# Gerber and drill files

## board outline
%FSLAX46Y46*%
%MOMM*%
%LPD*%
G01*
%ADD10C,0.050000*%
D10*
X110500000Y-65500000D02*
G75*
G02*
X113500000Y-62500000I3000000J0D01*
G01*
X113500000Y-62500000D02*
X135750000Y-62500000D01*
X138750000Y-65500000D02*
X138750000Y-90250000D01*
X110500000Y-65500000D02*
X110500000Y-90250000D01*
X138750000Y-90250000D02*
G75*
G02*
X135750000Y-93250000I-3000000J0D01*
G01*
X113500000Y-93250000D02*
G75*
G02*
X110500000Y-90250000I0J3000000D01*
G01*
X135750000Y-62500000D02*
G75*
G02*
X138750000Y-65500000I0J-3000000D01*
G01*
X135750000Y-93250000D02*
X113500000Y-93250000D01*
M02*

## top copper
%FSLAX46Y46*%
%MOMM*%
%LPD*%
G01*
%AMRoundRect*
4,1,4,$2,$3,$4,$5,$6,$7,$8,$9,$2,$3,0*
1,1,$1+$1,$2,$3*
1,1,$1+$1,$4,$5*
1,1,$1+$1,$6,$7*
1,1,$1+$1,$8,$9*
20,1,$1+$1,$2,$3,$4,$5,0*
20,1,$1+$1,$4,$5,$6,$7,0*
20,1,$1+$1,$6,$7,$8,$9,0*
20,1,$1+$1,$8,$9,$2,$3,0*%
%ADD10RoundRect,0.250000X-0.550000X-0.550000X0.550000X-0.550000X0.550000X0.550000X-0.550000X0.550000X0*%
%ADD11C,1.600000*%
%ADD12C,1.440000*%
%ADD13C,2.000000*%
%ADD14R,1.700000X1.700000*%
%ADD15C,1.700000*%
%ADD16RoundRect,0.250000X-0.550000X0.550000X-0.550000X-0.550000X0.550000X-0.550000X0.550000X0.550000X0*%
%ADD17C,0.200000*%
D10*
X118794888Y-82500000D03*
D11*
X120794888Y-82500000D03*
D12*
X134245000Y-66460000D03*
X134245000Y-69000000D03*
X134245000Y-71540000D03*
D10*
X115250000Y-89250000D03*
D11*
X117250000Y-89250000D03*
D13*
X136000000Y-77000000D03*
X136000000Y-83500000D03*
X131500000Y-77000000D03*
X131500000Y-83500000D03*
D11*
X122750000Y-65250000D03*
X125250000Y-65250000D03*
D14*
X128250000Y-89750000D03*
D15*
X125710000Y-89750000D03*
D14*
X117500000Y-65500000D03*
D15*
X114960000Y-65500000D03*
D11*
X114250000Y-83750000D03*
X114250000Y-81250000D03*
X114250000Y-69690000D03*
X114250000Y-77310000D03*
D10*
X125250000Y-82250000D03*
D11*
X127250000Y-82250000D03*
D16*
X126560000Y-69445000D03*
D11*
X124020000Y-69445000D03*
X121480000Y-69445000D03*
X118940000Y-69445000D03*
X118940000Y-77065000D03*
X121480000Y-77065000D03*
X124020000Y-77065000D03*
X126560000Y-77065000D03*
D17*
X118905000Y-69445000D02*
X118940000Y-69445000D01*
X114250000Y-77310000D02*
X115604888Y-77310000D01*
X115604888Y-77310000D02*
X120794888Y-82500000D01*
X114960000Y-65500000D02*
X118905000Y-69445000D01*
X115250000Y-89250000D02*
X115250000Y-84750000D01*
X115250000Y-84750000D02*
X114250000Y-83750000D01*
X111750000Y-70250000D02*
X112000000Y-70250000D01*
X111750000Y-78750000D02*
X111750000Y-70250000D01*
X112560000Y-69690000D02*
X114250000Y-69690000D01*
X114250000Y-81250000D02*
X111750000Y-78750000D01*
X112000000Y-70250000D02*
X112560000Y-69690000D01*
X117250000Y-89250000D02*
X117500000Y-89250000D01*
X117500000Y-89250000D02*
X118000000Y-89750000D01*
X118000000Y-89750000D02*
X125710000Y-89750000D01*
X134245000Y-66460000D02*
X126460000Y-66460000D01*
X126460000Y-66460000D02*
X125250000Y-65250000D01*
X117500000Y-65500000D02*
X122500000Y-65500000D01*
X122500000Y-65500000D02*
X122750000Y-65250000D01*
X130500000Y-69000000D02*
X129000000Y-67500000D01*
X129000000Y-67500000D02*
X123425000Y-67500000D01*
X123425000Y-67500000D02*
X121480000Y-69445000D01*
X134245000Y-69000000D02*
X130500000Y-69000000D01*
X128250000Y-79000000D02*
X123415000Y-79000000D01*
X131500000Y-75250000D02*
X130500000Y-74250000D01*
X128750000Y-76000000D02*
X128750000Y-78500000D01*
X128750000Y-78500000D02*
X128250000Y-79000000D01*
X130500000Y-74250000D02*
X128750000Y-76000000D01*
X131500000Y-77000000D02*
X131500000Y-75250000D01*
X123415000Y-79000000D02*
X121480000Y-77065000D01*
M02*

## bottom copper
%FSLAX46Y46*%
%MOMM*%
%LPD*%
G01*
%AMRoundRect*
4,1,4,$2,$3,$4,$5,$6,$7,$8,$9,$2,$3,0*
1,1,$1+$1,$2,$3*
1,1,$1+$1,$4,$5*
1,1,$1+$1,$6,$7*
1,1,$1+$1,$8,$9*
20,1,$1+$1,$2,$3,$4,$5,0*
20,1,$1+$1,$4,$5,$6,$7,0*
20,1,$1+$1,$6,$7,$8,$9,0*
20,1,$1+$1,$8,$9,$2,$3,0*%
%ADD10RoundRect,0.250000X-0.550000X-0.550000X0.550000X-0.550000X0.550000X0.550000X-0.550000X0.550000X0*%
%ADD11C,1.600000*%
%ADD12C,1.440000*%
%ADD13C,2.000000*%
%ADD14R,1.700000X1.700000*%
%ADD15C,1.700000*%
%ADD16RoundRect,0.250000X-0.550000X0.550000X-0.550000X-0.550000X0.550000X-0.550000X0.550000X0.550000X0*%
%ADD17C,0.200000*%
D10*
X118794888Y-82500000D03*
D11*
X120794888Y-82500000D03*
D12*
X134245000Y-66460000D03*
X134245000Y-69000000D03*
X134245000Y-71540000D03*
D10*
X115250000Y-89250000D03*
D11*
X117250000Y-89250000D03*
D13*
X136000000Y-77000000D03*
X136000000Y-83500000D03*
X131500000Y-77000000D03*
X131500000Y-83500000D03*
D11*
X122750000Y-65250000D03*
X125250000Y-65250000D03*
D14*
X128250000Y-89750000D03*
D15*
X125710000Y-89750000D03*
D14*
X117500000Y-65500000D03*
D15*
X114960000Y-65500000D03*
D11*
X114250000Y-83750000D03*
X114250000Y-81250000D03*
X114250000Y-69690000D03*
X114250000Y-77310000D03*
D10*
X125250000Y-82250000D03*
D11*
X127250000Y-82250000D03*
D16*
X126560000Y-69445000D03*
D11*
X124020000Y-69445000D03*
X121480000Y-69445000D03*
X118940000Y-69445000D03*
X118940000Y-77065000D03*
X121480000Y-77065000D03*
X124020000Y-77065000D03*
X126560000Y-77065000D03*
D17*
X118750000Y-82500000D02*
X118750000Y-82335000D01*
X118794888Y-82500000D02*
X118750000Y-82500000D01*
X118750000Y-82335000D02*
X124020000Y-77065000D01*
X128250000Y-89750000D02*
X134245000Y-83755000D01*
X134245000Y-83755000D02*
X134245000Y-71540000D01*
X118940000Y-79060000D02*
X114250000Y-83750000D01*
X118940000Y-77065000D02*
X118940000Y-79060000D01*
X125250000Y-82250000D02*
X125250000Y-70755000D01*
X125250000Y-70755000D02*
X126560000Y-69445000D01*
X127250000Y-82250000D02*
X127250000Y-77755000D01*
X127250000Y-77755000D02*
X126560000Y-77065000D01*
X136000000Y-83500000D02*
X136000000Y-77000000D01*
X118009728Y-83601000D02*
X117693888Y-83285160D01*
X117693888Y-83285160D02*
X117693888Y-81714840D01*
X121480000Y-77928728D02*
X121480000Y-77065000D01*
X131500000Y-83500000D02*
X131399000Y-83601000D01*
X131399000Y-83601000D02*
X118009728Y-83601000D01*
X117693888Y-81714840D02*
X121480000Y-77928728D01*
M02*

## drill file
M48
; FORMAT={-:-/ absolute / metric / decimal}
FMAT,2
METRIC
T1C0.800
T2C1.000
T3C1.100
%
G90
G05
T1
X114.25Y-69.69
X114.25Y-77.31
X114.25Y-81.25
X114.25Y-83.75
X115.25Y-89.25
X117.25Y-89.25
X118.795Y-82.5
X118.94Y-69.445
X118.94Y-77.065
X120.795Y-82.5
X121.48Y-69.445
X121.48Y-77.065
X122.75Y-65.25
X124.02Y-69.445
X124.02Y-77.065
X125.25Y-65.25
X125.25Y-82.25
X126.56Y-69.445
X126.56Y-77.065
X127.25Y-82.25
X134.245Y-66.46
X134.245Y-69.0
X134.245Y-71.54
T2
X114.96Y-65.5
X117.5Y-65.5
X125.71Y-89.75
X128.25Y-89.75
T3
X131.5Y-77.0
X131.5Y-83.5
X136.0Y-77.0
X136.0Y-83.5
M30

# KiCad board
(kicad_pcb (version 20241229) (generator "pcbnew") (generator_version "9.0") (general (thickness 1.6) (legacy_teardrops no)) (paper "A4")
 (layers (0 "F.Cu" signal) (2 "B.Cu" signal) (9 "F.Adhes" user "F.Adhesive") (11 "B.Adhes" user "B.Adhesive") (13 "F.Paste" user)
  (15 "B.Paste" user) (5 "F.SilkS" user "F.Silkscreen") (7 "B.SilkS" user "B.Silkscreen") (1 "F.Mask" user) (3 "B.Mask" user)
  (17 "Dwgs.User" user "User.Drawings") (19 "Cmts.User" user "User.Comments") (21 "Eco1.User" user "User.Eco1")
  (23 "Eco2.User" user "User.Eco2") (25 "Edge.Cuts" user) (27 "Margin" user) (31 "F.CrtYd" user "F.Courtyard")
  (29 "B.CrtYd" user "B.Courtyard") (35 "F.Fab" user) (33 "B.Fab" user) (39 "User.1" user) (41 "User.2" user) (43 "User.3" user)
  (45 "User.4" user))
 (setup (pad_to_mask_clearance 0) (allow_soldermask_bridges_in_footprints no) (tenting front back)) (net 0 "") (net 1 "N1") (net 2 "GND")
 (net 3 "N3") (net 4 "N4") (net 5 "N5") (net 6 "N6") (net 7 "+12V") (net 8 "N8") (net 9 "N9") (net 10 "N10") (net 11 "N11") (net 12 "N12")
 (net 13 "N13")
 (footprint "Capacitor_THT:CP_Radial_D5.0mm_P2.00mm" (layer "F.Cu") (at 118.794888 82.5)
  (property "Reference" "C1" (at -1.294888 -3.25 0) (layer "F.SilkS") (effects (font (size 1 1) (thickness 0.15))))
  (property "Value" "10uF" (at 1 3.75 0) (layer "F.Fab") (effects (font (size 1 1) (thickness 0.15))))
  (pad "1" thru_hole roundrect (at 0 0) (size 1.6 1.6) (drill 0.8) (layers "*.Cu" "*.Mask") (remove_unused_layers no)
   (roundrect_rratio 0.15625) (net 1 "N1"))
  (pad "2" thru_hole circle (at 2 0) (size 1.6 1.6) (drill 0.8) (layers "*.Cu" "*.Mask") (remove_unused_layers no) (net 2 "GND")))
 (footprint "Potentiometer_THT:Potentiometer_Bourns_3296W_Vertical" (layer "F.Cu") (at 134.245 66.46 90)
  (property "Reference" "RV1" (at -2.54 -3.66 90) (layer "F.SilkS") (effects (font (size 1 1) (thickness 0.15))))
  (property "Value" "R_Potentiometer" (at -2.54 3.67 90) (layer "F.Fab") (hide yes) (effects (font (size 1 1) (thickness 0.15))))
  (pad "1" thru_hole circle (at 0 0 90) (size 1.44 1.44) (drill 0.8) (layers "*.Cu" "*.Mask") (remove_unused_layers no) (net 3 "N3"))
  (pad "2" thru_hole circle (at -2.54 0 90) (size 1.44 1.44) (drill 0.8) (layers "*.Cu" "*.Mask") (remove_unused_layers no) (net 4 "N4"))
  (pad "3" thru_hole circle (at -5.08 0 90) (size 1.44 1.44) (drill 0.8) (layers "*.Cu" "*.Mask") (remove_unused_layers no) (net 2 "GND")))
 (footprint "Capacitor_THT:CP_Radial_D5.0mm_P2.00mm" (layer "F.Cu") (at 115.25 89.25)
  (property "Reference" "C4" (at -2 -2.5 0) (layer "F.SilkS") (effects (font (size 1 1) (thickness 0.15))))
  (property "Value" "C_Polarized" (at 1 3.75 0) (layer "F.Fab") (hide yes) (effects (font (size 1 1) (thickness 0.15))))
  (pad "1" thru_hole roundrect (at 0 0) (size 1.6 1.6) (drill 0.8) (layers "*.Cu" "*.Mask") (remove_unused_layers no)
   (roundrect_rratio 0.15625) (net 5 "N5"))
  (pad "2" thru_hole circle (at 2 0) (size 1.6 1.6) (drill 0.8) (layers "*.Cu" "*.Mask") (remove_unused_layers no) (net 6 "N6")))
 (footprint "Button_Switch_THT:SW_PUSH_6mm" (layer "F.Cu") (at 136 77 -90)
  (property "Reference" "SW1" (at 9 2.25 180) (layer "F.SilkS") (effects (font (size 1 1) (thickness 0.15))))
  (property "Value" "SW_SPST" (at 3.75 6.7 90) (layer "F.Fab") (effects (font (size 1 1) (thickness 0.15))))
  (pad "1" thru_hole circle (at 0 0) (size 2 2) (drill 1.1) (layers "*.Cu" "*.Mask") (remove_unused_layers no) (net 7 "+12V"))
  (pad "1" thru_hole circle (at 6.5 0) (size 2 2) (drill 1.1) (layers "*.Cu" "*.Mask") (remove_unused_layers no) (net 7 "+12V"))
  (pad "2" thru_hole circle (at 0 4.5) (size 2 2) (drill 1.1) (layers "*.Cu" "*.Mask") (remove_unused_layers no) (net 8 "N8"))
  (pad "2" thru_hole circle (at 6.5 4.5) (size 2 2) (drill 1.1) (layers "*.Cu" "*.Mask") (remove_unused_layers no) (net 8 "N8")))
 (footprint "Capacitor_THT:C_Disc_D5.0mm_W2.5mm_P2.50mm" (layer "F.Cu") (at 122.75 65.25)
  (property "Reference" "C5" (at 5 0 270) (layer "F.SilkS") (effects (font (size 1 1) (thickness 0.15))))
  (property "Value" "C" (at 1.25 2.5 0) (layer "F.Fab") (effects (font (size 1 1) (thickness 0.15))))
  (pad "1" thru_hole circle (at 0 0) (size 1.6 1.6) (drill 0.8) (layers "*.Cu" "*.Mask") (remove_unused_layers no) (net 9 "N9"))
  (pad "2" thru_hole circle (at 2.5 0) (size 1.6 1.6) (drill 0.8) (layers "*.Cu" "*.Mask") (remove_unused_layers no) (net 3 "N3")))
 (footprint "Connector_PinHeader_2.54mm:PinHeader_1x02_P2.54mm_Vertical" (layer "F.Cu") (at 128.25 89.75 -90)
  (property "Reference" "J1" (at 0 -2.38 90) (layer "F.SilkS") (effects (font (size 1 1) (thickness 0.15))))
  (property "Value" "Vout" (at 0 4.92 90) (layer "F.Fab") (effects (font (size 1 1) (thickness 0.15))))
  (pad "1" thru_hole rect (at 0 0 270) (size 1.7 1.7) (drill 1) (layers "*.Cu" "*.Mask") (remove_unused_layers no) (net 2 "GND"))
  (pad "2" thru_hole circle (at 0 2.54 270) (size 1.7 1.7) (drill 1) (layers "*.Cu" "*.Mask") (remove_unused_layers no) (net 6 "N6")))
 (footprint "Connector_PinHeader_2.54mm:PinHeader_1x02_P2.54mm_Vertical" (layer "F.Cu") (at 117.5 65.5 -90)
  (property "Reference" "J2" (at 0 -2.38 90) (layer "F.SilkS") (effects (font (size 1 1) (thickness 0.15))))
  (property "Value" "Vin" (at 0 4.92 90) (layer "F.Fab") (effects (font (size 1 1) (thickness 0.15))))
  (pad "1" thru_hole rect (at 0 0 270) (size 1.7 1.7) (drill 1) (layers "*.Cu" "*.Mask") (remove_unused_layers no) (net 9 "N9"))
  (pad "2" thru_hole circle (at 0 2.54 270) (size 1.7 1.7) (drill 1) (layers "*.Cu" "*.Mask") (remove_unused_layers no) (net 2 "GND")))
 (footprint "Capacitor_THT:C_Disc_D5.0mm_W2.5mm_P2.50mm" (layer "F.Cu") (at 114.25 83.75 90)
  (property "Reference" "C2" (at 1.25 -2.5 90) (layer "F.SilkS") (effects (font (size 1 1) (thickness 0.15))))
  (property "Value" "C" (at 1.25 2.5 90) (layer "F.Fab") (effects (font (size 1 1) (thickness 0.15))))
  (pad "1" thru_hole circle (at 0 0 90) (size 1.6 1.6) (drill 0.8) (layers "*.Cu" "*.Mask") (remove_unused_layers no) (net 5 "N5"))
  (pad "2" thru_hole circle (at 2.5 0 90) (size 1.6 1.6) (drill 0.8) (layers "*.Cu" "*.Mask") (remove_unused_layers no) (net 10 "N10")))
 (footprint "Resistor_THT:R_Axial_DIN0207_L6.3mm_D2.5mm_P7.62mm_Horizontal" (layer "F.Cu") (at 114.25 69.69 -90)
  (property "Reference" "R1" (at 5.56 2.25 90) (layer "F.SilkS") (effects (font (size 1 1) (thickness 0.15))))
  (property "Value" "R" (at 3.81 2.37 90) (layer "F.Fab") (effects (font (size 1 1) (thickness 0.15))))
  (pad "1" thru_hole circle (at 0 0 270) (size 1.6 1.6) (drill 0.8) (layers "*.Cu" "*.Mask") (remove_unused_layers no) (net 10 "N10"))
  (pad "2" thru_hole circle (at 7.62 0 270) (size 1.6 1.6) (drill 0.8) (layers "*.Cu" "*.Mask") (remove_unused_layers no) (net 2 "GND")))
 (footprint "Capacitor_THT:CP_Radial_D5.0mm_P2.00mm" (layer "F.Cu") (at 125.25 82.25)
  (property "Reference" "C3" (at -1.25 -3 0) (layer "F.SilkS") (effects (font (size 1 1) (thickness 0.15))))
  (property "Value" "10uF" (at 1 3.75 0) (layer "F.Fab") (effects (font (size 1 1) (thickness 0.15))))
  (pad "1" thru_hole roundrect (at 0 0) (size 1.6 1.6) (drill 0.8) (layers "*.Cu" "*.Mask") (remove_unused_layers no)
   (roundrect_rratio 0.15625) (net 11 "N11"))
  (pad "2" thru_hole circle (at 2 0) (size 1.6 1.6) (drill 0.8) (layers "*.Cu" "*.Mask") (remove_unused_layers no) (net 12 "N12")))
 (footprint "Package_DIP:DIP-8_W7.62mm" (layer "F.Cu") (at 126.56 69.445 -90)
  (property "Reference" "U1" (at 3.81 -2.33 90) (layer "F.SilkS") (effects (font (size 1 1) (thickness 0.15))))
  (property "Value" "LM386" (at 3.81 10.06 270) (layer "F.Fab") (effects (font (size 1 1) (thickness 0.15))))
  (pad "1" thru_hole roundrect (at 0 0 270) (size 1.6 1.6) (drill 0.8) (layers "*.Cu" "*.Mask") (remove_unused_layers no)
   (roundrect_rratio 0.15625) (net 11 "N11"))
  (pad "2" thru_hole circle (at 0 2.54 270) (size 1.6 1.6) (drill 0.8) (layers "*.Cu" "*.Mask") (remove_unused_layers no) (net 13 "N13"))
  (pad "3" thru_hole circle (at 0 5.08 270) (size 1.6 1.6) (drill 0.8) (layers "*.Cu" "*.Mask") (remove_unused_layers no) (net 4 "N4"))
  (pad "4" thru_hole circle (at 0 7.62 270) (size 1.6 1.6) (drill 0.8) (layers "*.Cu" "*.Mask") (remove_unused_layers no) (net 2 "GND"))
  (pad "5" thru_hole circle (at 7.62 7.62 270) (size 1.6 1.6) (drill 0.8) (layers "*.Cu" "*.Mask") (remove_unused_layers no) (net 5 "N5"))
  (pad "6" thru_hole circle (at 7.62 5.08 270) (size 1.6 1.6) (drill 0.8) (layers "*.Cu" "*.Mask") (remove_unused_layers no) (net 8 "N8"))
  (pad "7" thru_hole circle (at 7.62 2.54 270) (size 1.6 1.6) (drill 0.8) (layers "*.Cu" "*.Mask") (remove_unused_layers no) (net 1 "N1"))
  (pad "8" thru_hole circle (at 7.62 0 270) (size 1.6 1.6) (drill 0.8) (layers "*.Cu" "*.Mask") (remove_unused_layers no) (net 12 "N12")))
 (gr_arc (start 110.5 65.5) (mid 111.37868 63.37868) (end 113.5 62.5) (stroke (width 0.05) (type default)) (layer "Edge.Cuts"))
 (gr_line (start 113.5 62.5) (end 135.75 62.5) (stroke (width 0.05) (type default)) (layer "Edge.Cuts"))
 (gr_line (start 138.75 65.5) (end 138.75 90.25) (stroke (width 0.05) (type default)) (layer "Edge.Cuts"))
 (gr_line (start 110.5 65.5) (end 110.5 90.25) (stroke (width 0.05) (type default)) (layer "Edge.Cuts"))
 (gr_arc (start 138.75 90.25) (mid 137.87132 92.37132) (end 135.75 93.25) (stroke (width 0.05) (type default)) (layer "Edge.Cuts"))
 (gr_arc (start 113.5 93.25) (mid 111.37868 92.37132) (end 110.5 90.25) (stroke (width 0.05) (type default)) (layer "Edge.Cuts"))
 (gr_arc (start 135.75 62.5) (mid 137.87132 63.37868) (end 138.75 65.5) (stroke (width 0.05) (type default)) (layer "Edge.Cuts"))
 (gr_line (start 135.75 93.25) (end 113.5 93.25) (stroke (width 0.05) (type default)) (layer "Edge.Cuts"))
 (segment (start 118.75 82.5) (end 118.75 82.335) (width 0.2) (layer "B.Cu") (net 1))
 (segment (start 118.794888 82.5) (end 118.75 82.5) (width 0.2) (layer "B.Cu") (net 1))
 (segment (start 118.75 82.335) (end 124.02 77.065) (width 0.2) (layer "B.Cu") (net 1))
 (segment (start 118.905 69.445) (end 118.94 69.445) (width 0.2) (layer "F.Cu") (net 2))
 (segment (start 114.25 77.31) (end 115.604888 77.31) (width 0.2) (layer "F.Cu") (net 2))
 (segment (start 115.604888 77.31) (end 120.794888 82.5) (width 0.2) (layer "F.Cu") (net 2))
 (segment (start 114.96 65.5) (end 118.905 69.445) (width 0.2) (layer "F.Cu") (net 2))
 (segment (start 128.25 89.75) (end 134.245 83.755) (width 0.2) (layer "B.Cu") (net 2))
 (segment (start 134.245 83.755) (end 134.245 71.54) (width 0.2) (layer "B.Cu") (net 2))
 (segment (start 115.25 89.25) (end 115.25 84.75) (width 0.2) (layer "F.Cu") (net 5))
 (segment (start 115.25 84.75) (end 114.25 83.75) (width 0.2) (layer "F.Cu") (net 5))
 (segment (start 118.94 79.06) (end 114.25 83.75) (width 0.2) (layer "B.Cu") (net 5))
 (segment (start 118.94 77.065) (end 118.94 79.06) (width 0.2) (layer "B.Cu") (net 5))
 (segment (start 111.75 70.25) (end 112 70.25) (width 0.2) (layer "F.Cu") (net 10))
 (segment (start 111.75 78.75) (end 111.75 70.25) (width 0.2) (layer "F.Cu") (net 10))
 (segment (start 112.56 69.69) (end 114.25 69.69) (width 0.2) (layer "F.Cu") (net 10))
 (segment (start 114.25 81.25) (end 111.75 78.75) (width 0.2) (layer "F.Cu") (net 10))
 (segment (start 112 70.25) (end 112.56 69.69) (width 0.2) (layer "F.Cu") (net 10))
 (segment (start 125.25 82.25) (end 125.25 70.755) (width 0.2) (layer "B.Cu") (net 11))
 (segment (start 125.25 70.755) (end 126.56 69.445) (width 0.2) (layer "B.Cu") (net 11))
 (segment (start 127.25 82.25) (end 127.25 77.755) (width 0.2) (layer "B.Cu") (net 12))
 (segment (start 127.25 77.755) (end 126.56 77.065) (width 0.2) (layer "B.Cu") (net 12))
 (segment (start 117.25 89.25) (end 117.5 89.25) (width 0.2) (layer "F.Cu") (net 6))
 (segment (start 117.5 89.25) (end 118 89.75) (width 0.2) (layer "F.Cu") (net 6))
 (segment (start 118 89.75) (end 125.71 89.75) (width 0.2) (layer "F.Cu") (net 6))
 (segment (start 134.245 66.46) (end 126.46 66.46) (width 0.2) (layer "F.Cu") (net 3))
 (segment (start 126.46 66.46) (end 125.25 65.25) (width 0.2) (layer "F.Cu") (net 3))
 (segment (start 117.5 65.5) (end 122.5 65.5) (width 0.2) (layer "F.Cu") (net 9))
 (segment (start 122.5 65.5) (end 122.75 65.25) (width 0.2) (layer "F.Cu") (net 9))
 (segment (start 130.5 69) (end 129 67.5) (width 0.2) (layer "F.Cu") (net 4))
 (segment (start 129 67.5) (end 123.425 67.5) (width 0.2) (layer "F.Cu") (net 4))
 (segment (start 123.425 67.5) (end 121.48 69.445) (width 0.2) (layer "F.Cu") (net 4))
 (segment (start 134.245 69) (end 130.5 69) (width 0.2) (layer "F.Cu") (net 4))
 (segment (start 136 83.5) (end 136 77) (width 0.2) (layer "B.Cu") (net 7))
 (segment (start 128.25 79) (end 123.415 79) (width 0.2) (layer "F.Cu") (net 8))
 (segment (start 131.5 75.25) (end 130.5 74.25) (width 0.2) (layer "F.Cu") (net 8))
 (segment (start 128.75 76) (end 128.75 78.5) (width 0.2) (layer "F.Cu") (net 8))
 (segment (start 128.75 78.5) (end 128.25 79) (width 0.2) (layer "F.Cu") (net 8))
 (segment (start 130.5 74.25) (end 128.75 76) (width 0.2) (layer "F.Cu") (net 8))
 (segment (start 131.5 77) (end 131.5 75.25) (width 0.2) (layer "F.Cu") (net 8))
 (segment (start 123.415 79) (end 121.48 77.065) (width 0.2) (layer "F.Cu") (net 8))
 (segment (start 118.009728 83.601) (end 117.693888 83.28516) (width 0.2) (layer "B.Cu") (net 8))
 (segment (start 117.693888 83.28516) (end 117.693888 81.71484) (width 0.2) (layer "B.Cu") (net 8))
 (segment (start 121.48 77.928728) (end 121.48 77.065) (width 0.2) (layer "B.Cu") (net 8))
 (segment (start 131.5 83.5) (end 131.399 83.601) (width 0.2) (layer "B.Cu") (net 8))
 (segment (start 131.399 83.601) (end 118.009728 83.601) (width 0.2) (layer "B.Cu") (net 8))
 (segment (start 117.693888 81.71484) (end 121.48 77.928728) (width 0.2) (layer "B.Cu") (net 8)))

